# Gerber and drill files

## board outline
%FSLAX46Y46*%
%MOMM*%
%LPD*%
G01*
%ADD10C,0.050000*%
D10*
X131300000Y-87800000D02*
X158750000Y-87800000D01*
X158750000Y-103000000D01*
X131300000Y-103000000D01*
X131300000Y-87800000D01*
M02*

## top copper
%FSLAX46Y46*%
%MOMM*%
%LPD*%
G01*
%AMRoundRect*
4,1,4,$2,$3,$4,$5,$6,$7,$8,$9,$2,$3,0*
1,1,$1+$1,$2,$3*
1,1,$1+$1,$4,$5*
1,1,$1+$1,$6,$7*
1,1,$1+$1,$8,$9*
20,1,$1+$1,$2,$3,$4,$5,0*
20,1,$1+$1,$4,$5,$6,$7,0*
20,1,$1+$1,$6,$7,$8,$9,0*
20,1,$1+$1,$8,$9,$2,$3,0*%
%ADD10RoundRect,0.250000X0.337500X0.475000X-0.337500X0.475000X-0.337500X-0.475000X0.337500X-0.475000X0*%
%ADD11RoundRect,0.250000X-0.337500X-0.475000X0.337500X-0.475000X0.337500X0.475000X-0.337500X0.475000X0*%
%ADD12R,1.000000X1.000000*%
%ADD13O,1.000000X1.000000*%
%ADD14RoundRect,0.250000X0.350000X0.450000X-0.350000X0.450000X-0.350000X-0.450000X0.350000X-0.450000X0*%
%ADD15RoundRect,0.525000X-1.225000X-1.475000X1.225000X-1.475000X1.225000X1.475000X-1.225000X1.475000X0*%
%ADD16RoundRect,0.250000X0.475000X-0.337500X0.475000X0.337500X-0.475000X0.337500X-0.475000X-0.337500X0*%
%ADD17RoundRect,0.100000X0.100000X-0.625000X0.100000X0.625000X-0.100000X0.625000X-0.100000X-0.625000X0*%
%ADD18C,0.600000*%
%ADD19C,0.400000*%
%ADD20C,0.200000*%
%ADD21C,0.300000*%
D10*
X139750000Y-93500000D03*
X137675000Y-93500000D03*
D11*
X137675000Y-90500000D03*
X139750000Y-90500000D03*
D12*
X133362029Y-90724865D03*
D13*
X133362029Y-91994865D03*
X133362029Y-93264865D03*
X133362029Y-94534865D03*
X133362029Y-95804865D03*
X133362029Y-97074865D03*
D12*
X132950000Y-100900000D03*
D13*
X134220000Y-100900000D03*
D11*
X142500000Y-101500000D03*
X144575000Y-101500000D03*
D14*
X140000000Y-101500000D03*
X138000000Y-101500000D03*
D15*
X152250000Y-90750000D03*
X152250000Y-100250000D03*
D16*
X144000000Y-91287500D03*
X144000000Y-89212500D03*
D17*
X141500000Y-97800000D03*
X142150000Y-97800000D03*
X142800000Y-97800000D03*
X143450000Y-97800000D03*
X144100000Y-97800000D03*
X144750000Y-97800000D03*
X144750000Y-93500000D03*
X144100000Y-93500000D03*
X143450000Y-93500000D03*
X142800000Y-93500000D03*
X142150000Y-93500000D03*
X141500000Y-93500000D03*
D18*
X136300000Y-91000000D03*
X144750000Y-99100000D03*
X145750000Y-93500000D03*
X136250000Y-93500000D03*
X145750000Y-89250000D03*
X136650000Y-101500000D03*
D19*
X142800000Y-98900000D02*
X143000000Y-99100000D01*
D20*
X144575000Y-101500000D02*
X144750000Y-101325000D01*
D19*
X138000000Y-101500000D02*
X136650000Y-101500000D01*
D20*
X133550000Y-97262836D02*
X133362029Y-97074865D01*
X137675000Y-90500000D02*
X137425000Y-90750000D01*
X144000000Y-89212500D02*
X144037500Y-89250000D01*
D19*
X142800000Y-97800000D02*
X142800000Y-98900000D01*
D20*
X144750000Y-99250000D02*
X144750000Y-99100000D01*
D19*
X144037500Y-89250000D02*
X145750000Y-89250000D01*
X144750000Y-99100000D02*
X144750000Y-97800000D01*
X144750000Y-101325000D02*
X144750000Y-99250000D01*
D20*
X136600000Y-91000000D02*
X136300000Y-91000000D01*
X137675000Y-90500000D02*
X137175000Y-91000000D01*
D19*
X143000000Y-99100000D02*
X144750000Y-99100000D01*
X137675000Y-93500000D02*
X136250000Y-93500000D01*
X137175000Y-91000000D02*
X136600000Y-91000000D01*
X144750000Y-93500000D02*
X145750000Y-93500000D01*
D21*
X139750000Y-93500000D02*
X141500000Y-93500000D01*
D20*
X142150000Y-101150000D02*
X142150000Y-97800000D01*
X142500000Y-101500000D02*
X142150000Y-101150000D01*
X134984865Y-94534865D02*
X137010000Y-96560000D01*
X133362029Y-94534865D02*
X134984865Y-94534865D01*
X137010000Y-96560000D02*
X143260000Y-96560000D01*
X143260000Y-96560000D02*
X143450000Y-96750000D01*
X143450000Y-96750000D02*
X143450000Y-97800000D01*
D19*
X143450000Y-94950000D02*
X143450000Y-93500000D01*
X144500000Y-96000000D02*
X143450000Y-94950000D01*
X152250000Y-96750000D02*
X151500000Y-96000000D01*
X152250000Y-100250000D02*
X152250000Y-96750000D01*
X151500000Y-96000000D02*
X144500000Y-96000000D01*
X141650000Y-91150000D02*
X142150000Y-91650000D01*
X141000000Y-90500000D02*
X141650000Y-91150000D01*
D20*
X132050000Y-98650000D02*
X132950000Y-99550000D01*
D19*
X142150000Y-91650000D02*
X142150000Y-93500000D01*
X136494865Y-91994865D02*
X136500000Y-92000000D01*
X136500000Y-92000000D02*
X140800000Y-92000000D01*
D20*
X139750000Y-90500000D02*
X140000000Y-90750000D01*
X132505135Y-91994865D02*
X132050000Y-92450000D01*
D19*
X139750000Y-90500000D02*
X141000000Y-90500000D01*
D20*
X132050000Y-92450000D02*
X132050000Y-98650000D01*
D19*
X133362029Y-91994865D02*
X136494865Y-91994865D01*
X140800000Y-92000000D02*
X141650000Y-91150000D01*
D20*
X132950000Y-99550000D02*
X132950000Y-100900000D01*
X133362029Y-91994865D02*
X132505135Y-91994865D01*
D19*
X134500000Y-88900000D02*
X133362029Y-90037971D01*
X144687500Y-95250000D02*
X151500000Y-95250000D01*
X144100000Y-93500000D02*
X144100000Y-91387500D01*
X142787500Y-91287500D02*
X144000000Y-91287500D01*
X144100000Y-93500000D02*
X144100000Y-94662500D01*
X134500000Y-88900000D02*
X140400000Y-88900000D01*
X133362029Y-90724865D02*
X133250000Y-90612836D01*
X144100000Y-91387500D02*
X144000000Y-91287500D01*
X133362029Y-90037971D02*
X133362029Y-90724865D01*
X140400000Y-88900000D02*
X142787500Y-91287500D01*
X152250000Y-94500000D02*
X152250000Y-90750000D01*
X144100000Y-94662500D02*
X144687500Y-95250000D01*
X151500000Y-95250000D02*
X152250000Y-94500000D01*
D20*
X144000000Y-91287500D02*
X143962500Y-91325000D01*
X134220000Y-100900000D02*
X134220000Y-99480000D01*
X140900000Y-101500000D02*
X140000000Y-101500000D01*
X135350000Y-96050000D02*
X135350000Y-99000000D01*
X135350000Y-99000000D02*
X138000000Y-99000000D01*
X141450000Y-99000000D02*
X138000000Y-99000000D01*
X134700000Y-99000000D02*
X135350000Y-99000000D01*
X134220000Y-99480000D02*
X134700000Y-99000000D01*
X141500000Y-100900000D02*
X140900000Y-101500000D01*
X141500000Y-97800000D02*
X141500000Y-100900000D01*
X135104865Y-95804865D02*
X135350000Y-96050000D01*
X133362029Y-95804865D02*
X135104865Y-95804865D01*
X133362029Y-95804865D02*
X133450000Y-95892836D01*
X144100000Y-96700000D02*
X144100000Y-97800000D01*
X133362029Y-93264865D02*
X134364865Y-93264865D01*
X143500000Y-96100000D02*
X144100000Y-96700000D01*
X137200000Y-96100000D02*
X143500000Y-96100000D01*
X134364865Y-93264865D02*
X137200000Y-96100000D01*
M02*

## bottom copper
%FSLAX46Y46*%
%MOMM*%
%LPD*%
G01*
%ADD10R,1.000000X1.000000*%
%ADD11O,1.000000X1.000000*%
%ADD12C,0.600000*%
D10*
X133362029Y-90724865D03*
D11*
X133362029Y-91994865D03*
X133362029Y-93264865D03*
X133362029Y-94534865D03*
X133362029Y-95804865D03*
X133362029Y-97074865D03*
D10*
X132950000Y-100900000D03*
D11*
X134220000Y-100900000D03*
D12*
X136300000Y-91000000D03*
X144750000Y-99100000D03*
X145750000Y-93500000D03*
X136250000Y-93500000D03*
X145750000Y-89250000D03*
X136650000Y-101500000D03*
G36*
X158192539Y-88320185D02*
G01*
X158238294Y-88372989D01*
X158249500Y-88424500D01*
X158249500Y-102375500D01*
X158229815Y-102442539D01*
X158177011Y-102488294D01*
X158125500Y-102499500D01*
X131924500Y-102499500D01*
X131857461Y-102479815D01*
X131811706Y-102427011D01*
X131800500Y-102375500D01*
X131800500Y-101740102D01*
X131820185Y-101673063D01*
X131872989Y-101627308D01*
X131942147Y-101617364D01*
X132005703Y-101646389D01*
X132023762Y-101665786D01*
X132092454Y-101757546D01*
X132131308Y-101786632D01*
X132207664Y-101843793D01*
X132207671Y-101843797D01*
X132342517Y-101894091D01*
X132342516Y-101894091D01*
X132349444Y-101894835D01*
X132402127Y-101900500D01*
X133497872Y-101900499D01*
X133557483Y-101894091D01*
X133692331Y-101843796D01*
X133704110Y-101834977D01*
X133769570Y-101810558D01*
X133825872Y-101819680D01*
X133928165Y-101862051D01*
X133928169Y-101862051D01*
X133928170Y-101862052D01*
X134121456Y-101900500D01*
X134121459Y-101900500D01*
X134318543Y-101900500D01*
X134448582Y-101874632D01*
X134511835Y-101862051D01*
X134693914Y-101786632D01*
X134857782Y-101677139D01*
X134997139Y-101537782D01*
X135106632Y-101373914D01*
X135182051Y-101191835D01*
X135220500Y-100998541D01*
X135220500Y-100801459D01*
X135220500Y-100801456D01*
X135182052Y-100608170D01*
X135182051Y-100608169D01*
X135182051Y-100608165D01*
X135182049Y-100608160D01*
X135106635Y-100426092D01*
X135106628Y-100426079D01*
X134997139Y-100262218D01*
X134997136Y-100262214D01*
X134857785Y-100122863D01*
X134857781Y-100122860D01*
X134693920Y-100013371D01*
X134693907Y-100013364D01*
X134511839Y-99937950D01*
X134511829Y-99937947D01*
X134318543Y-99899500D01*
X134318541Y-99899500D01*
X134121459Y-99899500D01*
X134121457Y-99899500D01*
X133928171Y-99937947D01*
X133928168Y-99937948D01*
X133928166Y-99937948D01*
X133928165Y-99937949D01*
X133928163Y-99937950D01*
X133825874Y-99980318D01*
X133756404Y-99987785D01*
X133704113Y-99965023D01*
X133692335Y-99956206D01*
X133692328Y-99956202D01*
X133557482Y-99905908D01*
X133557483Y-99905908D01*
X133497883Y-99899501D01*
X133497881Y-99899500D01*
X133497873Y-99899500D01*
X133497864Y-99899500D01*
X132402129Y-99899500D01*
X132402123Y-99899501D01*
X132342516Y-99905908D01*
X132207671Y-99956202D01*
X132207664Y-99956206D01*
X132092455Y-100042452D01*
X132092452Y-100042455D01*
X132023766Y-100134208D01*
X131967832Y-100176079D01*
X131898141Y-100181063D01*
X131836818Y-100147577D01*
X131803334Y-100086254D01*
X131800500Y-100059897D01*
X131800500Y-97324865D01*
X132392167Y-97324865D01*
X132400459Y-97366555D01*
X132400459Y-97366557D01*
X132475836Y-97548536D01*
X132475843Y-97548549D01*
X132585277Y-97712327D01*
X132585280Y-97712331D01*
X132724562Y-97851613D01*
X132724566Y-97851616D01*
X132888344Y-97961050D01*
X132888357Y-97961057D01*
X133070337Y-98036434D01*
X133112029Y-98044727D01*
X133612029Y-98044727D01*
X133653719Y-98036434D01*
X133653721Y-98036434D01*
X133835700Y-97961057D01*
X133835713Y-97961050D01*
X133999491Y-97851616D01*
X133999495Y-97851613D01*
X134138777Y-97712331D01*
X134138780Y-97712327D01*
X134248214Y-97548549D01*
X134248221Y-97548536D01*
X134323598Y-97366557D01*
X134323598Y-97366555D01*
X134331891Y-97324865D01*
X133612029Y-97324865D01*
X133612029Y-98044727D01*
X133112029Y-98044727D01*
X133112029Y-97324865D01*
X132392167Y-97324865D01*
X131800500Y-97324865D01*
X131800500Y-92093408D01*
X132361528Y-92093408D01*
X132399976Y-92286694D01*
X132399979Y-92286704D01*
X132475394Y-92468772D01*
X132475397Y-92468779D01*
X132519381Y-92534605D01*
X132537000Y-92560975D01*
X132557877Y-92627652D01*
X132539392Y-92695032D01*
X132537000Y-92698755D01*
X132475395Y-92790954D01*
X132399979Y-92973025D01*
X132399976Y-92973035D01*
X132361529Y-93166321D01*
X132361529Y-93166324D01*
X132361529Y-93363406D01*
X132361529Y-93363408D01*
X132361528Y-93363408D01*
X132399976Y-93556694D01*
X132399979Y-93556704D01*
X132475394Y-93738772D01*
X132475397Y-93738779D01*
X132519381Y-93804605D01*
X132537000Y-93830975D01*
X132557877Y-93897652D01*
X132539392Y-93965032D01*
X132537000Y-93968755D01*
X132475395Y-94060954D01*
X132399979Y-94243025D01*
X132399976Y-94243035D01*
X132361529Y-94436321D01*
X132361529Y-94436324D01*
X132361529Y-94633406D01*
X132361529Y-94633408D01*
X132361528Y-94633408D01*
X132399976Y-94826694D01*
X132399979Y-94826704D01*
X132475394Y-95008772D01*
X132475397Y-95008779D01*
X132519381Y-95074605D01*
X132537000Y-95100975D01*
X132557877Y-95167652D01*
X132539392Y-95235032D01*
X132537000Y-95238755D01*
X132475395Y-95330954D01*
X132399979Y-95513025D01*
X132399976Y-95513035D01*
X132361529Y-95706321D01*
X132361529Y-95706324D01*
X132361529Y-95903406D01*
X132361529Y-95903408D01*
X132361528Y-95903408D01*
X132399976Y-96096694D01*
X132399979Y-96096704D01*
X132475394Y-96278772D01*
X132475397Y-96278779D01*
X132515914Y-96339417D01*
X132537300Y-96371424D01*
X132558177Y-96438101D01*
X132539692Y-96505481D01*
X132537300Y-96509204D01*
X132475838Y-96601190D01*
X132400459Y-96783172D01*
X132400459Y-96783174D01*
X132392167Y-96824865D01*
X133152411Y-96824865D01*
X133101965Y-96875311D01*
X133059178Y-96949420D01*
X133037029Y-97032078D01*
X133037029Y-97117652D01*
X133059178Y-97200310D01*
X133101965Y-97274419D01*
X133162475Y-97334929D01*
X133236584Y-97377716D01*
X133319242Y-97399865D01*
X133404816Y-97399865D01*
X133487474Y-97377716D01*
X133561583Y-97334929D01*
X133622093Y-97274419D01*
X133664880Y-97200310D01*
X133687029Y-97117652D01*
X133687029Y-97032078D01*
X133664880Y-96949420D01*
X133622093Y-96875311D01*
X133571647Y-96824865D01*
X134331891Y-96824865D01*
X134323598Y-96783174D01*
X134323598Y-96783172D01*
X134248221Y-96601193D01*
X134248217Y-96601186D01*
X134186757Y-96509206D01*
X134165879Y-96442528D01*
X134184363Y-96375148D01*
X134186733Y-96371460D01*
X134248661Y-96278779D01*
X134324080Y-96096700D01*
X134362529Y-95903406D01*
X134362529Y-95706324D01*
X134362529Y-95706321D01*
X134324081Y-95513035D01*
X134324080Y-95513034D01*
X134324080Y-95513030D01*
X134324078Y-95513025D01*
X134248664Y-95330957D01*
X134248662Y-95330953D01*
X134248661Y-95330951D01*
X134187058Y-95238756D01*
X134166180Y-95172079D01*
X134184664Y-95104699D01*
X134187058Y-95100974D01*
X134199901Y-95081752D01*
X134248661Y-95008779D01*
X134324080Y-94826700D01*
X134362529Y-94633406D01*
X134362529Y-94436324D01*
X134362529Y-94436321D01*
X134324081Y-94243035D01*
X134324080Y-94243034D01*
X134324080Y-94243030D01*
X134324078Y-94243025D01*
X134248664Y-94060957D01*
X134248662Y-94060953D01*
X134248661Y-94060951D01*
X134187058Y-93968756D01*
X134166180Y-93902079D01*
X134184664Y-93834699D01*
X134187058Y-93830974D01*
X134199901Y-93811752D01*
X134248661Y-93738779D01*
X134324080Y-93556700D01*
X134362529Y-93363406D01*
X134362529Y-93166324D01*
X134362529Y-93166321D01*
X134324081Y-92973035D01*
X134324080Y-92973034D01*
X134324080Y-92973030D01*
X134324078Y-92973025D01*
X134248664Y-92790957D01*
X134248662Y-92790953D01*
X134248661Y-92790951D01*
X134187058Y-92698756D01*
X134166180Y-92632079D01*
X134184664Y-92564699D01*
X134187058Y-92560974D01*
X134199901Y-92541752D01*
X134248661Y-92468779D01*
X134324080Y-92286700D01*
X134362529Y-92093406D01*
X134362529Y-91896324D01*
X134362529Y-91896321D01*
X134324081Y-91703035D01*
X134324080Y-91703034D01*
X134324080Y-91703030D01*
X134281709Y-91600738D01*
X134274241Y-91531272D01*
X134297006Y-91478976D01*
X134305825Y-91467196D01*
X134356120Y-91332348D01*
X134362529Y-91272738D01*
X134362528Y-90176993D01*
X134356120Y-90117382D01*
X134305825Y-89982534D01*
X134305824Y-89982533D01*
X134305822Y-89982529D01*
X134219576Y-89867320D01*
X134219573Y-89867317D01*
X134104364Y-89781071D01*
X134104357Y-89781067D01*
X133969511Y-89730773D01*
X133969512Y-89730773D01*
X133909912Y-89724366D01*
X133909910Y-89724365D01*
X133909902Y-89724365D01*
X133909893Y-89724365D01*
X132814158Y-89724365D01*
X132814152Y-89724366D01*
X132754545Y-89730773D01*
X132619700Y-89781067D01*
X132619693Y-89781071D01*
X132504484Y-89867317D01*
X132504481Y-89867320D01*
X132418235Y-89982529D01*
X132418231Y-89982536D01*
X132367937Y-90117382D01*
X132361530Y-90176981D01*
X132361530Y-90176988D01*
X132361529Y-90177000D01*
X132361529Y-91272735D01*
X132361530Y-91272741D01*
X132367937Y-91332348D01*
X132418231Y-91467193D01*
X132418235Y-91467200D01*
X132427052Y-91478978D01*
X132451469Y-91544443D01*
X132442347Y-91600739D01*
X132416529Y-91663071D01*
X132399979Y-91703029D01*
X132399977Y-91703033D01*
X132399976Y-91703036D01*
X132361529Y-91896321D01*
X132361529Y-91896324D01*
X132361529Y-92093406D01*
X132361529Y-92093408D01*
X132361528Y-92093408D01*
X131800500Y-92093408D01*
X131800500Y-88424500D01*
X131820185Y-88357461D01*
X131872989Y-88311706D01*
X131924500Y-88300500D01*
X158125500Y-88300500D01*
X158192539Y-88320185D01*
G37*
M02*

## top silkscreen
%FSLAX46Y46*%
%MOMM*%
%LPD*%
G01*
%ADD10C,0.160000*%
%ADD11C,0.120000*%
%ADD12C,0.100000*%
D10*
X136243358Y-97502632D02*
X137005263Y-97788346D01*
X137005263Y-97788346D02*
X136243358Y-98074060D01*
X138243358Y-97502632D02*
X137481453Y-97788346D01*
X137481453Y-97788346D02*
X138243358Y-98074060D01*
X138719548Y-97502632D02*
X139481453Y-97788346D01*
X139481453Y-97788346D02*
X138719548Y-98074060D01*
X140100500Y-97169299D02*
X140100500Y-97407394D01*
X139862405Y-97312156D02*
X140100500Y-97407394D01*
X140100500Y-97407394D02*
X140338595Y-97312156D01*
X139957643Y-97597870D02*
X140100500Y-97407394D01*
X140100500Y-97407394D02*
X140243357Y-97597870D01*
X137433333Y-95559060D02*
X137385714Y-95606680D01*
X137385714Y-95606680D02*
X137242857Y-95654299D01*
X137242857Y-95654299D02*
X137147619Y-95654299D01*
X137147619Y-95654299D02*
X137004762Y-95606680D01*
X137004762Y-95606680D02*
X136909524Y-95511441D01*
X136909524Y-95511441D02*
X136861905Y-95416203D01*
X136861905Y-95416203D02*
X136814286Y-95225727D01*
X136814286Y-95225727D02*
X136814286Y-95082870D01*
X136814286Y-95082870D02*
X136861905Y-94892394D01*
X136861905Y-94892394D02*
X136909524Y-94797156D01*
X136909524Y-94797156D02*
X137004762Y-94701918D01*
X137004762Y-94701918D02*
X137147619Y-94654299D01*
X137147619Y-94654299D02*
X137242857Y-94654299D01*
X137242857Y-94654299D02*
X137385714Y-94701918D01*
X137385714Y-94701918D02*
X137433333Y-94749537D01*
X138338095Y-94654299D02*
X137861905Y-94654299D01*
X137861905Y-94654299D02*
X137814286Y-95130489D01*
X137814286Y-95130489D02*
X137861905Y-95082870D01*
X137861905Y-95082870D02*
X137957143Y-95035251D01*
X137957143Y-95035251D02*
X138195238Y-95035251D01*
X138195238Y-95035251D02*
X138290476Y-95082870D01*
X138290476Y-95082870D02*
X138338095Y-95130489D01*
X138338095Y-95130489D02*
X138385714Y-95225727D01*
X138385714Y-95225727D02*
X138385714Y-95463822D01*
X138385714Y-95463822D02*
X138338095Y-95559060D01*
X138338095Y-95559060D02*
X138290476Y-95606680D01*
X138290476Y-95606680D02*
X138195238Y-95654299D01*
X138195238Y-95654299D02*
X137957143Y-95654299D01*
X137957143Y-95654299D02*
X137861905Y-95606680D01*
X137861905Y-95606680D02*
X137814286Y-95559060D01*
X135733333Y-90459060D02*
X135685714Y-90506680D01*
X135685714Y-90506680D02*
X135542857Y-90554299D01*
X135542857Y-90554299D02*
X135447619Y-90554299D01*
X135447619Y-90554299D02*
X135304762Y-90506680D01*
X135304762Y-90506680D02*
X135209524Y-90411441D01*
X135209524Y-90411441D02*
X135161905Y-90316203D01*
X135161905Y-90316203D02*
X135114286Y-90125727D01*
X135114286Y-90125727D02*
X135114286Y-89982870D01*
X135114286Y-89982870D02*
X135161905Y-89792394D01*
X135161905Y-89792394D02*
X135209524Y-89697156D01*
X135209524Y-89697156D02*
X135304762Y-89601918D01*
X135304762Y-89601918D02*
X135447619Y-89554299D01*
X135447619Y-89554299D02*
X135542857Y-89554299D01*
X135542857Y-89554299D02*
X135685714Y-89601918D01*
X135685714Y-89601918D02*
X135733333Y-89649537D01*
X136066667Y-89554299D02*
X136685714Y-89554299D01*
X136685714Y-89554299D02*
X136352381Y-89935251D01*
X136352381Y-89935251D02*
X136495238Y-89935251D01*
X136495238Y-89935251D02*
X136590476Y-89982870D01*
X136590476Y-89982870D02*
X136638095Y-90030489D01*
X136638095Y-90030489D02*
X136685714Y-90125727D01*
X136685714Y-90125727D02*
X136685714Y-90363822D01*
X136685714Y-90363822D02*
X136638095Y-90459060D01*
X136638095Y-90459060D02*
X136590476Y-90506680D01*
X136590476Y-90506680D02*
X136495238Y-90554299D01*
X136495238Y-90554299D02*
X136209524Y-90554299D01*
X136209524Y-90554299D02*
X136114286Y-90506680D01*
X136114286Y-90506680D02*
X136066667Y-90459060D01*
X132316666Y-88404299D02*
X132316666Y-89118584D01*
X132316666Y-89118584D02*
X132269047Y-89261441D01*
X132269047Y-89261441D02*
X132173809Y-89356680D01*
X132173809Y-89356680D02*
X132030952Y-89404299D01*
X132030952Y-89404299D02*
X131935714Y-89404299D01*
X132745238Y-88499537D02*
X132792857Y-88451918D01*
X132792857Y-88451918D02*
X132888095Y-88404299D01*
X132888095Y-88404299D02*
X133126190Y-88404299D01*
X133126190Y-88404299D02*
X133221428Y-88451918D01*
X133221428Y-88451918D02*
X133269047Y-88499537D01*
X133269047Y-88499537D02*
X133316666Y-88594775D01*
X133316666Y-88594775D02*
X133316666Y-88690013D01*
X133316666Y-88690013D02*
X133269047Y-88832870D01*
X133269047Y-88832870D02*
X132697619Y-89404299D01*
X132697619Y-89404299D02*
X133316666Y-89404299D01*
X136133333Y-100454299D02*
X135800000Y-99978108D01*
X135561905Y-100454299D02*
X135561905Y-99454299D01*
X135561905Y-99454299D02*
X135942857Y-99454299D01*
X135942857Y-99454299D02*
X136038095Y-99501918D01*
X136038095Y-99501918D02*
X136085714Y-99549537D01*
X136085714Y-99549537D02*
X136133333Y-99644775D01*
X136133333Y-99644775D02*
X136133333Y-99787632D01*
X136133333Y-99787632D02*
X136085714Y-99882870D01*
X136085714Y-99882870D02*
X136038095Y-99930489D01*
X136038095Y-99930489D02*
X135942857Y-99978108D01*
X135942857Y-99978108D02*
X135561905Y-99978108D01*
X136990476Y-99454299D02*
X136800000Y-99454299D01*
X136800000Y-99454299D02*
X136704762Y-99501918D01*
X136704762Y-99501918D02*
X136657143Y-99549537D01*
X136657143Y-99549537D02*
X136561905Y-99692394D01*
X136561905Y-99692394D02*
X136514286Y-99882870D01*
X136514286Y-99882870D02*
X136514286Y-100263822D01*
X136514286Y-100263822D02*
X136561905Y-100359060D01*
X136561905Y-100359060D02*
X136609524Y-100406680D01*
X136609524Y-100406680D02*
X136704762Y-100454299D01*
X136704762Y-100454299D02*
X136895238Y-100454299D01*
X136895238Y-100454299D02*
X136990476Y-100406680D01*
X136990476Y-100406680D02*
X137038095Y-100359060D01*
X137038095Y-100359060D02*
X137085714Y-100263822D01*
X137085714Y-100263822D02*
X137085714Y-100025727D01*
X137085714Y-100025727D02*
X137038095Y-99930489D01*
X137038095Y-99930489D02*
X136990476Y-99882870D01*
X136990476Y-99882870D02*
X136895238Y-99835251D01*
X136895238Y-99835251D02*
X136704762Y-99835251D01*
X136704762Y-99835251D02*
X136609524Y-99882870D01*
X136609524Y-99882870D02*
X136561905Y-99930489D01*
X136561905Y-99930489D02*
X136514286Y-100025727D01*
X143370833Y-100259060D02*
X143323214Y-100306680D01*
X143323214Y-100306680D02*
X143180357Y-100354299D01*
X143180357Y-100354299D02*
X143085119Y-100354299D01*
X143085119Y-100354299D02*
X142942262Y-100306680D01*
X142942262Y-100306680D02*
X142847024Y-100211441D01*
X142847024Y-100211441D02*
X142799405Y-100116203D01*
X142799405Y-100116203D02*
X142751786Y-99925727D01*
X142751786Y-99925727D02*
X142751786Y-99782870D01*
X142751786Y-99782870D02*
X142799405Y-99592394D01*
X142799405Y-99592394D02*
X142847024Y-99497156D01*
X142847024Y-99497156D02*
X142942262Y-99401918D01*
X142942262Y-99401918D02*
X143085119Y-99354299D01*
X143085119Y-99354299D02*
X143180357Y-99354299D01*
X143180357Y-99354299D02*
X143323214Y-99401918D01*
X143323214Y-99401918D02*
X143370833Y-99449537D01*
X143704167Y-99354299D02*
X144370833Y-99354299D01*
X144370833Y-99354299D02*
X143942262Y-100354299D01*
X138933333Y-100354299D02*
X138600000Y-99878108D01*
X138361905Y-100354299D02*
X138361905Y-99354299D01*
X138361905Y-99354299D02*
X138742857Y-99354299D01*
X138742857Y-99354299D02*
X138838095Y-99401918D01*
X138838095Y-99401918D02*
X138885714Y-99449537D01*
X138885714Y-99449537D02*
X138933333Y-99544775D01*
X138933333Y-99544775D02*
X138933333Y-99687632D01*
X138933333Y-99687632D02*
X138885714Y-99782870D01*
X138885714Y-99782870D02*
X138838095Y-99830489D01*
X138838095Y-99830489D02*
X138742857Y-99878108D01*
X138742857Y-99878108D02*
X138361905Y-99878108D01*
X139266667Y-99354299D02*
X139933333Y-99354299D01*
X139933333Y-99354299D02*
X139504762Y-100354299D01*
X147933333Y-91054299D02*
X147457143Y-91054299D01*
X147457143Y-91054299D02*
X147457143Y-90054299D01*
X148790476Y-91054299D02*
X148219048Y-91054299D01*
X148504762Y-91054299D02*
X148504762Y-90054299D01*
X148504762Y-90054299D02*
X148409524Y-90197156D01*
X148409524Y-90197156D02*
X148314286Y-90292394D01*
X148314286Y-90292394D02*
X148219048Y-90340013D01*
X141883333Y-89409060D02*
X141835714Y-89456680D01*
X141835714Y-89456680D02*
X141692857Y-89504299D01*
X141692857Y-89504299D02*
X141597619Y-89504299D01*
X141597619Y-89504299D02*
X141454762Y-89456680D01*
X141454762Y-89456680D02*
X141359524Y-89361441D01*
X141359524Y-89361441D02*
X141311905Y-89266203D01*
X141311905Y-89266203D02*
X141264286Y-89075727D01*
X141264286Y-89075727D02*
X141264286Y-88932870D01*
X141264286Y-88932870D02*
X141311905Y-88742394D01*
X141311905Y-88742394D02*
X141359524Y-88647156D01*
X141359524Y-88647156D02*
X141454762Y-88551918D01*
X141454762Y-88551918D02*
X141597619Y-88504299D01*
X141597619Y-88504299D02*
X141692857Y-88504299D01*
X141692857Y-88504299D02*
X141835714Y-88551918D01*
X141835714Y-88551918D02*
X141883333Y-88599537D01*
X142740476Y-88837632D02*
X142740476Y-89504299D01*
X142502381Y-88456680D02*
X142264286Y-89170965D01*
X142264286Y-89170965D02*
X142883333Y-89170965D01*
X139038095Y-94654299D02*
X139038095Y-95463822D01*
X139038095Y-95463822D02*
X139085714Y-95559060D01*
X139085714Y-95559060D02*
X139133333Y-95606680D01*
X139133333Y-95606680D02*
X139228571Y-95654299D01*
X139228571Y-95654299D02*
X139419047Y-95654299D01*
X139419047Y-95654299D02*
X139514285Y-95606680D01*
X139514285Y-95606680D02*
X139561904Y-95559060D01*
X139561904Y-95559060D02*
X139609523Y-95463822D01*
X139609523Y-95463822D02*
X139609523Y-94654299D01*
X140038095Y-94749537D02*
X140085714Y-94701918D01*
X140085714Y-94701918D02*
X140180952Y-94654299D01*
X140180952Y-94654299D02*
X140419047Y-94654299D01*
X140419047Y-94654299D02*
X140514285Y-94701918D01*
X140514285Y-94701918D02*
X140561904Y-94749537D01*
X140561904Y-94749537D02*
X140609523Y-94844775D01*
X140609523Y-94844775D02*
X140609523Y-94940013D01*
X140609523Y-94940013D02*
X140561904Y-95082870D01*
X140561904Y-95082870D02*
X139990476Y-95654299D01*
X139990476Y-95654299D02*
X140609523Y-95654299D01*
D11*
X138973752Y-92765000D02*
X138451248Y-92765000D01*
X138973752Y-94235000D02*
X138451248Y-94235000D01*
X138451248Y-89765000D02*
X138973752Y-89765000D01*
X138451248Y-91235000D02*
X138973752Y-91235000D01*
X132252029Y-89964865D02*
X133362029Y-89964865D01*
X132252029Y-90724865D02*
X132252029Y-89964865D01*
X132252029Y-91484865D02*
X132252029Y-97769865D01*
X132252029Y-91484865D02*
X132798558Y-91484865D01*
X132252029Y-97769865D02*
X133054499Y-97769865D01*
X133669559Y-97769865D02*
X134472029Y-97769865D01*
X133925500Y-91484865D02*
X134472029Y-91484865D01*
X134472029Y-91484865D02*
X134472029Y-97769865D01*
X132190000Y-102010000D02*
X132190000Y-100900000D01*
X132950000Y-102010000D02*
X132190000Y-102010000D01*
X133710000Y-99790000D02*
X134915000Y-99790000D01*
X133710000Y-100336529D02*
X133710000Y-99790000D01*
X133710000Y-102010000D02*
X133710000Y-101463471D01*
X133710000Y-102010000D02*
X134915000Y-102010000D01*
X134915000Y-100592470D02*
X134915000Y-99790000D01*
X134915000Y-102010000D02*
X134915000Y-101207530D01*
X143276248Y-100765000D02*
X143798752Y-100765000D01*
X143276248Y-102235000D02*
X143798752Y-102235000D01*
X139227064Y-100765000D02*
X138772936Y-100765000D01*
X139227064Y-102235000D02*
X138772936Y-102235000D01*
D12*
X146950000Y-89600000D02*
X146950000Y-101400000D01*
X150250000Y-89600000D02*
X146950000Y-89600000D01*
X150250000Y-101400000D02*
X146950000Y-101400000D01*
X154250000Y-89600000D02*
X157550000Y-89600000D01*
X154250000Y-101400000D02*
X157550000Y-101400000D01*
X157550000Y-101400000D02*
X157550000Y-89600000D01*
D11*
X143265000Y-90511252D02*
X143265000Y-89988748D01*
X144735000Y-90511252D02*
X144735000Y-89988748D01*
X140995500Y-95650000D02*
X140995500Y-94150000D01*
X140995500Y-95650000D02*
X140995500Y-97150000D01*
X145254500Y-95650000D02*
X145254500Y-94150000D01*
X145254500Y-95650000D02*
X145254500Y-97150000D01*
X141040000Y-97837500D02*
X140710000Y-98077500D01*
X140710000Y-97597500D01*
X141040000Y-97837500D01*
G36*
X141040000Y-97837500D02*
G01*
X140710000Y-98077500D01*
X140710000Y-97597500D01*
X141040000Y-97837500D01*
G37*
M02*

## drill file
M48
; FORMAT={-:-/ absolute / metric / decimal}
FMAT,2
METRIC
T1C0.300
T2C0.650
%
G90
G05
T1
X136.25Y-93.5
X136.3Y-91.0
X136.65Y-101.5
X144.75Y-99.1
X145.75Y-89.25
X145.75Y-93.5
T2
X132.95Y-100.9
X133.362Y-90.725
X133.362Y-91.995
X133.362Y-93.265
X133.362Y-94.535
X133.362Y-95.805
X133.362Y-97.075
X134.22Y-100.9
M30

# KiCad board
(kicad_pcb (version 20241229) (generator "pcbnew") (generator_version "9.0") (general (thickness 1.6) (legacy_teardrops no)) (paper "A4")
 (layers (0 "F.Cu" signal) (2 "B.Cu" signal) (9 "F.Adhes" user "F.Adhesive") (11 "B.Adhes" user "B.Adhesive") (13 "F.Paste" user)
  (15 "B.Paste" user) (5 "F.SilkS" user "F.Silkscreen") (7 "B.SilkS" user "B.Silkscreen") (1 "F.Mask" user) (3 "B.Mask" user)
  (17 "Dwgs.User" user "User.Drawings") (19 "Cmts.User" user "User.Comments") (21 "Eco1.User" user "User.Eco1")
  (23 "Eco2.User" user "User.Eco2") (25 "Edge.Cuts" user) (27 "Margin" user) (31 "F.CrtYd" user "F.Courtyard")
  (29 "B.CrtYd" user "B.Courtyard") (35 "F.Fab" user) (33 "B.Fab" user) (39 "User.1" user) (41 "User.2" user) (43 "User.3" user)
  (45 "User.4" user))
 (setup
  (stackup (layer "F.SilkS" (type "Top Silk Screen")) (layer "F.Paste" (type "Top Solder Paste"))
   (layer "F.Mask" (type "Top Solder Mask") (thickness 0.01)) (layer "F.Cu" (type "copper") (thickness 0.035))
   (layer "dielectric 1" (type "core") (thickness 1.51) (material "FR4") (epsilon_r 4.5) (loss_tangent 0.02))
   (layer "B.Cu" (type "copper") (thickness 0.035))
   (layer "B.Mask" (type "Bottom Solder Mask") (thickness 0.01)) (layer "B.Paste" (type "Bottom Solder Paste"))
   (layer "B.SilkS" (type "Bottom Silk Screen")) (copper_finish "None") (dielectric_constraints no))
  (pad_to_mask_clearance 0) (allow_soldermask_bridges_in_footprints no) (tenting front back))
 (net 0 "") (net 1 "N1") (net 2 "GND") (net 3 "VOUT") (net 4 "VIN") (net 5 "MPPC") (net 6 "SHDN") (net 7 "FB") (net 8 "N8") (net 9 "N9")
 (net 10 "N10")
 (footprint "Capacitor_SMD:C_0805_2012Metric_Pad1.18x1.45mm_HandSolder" (layer "F.Cu") (at 138.7125 93.5 180)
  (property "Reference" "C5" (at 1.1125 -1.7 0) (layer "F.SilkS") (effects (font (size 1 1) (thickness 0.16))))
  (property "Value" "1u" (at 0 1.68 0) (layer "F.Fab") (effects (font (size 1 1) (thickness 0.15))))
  (fp_line (start -0.261252 0.735) (end 0.261252 0.735) (stroke (width 0.12) (type solid)) (layer "F.SilkS"))
  (fp_line (start -0.261252 -0.735) (end 0.261252 -0.735) (stroke (width 0.12) (type solid)) (layer "F.SilkS"))
  (pad "1" smd roundrect (at -1.0375 0 180) (size 1.175 1.45) (layers "F.Cu" "F.Mask" "F.Paste") (roundrect_rratio 0.212766) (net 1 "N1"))
  (pad "2" smd roundrect (at 1.0375 0 180) (size 1.175 1.45) (layers "F.Cu" "F.Mask" "F.Paste") (roundrect_rratio 0.212766) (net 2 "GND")))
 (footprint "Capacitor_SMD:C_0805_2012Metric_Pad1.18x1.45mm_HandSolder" (layer "F.Cu") (at 138.7125 90.5)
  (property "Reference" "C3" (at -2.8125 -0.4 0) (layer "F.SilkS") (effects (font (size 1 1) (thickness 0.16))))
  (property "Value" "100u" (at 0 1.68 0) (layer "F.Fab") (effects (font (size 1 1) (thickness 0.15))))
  (fp_line (start -0.261252 -0.735) (end 0.261252 -0.735) (stroke (width 0.12) (type solid)) (layer "F.SilkS"))
  (fp_line (start -0.261252 0.735) (end 0.261252 0.735) (stroke (width 0.12) (type solid)) (layer "F.SilkS"))
  (pad "1" smd roundrect (at -1.0375 0) (size 1.175 1.45) (layers "F.Cu" "F.Mask" "F.Paste") (roundrect_rratio 0.212766) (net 2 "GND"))
  (pad "2" smd roundrect (at 1.0375 0) (size 1.175 1.45) (layers "F.Cu" "F.Mask" "F.Paste") (roundrect_rratio 0.212766) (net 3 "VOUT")))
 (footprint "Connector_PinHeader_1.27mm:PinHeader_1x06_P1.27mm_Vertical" (layer "F.Cu") (at 133.362029 90.724865)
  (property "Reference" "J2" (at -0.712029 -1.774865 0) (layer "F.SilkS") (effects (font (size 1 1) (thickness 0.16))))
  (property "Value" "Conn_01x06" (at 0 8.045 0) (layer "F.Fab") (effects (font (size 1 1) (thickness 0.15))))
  (fp_line (start -1.11 -0.76) (end 0 -0.76) (stroke (width 0.12) (type solid)) (layer "F.SilkS"))
  (fp_line (start -1.11 0) (end -1.11 -0.76) (stroke (width 0.12) (type solid)) (layer "F.SilkS"))
  (fp_line (start -1.11 0.76) (end -1.11 7.045) (stroke (width 0.12) (type solid)) (layer "F.SilkS"))
  (fp_line (start -1.11 0.76) (end -0.563471 0.76) (stroke (width 0.12) (type solid)) (layer "F.SilkS"))
  (fp_line (start -1.11 7.045) (end -0.30753 7.045) (stroke (width 0.12) (type solid)) (layer "F.SilkS"))
  (fp_line (start 0.30753 7.045) (end 1.11 7.045) (stroke (width 0.12) (type solid)) (layer "F.SilkS"))
  (fp_line (start 0.563471 0.76) (end 1.11 0.76) (stroke (width 0.12) (type solid)) (layer "F.SilkS"))
  (fp_line (start 1.11 0.76) (end 1.11 7.045) (stroke (width 0.12) (type solid)) (layer "F.SilkS"))
  (pad "1" thru_hole rect (at 0 0) (size 1 1) (drill 0.65) (layers "*.Cu" "*.Mask") (remove_unused_layers no) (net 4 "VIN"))
  (pad "2" thru_hole oval (at 0 1.27) (size 1 1) (drill 0.65) (layers "*.Cu" "*.Mask") (remove_unused_layers no) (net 3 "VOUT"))
  (pad "3" thru_hole oval (at 0 2.54) (size 1 1) (drill 0.65) (layers "*.Cu" "*.Mask") (remove_unused_layers no) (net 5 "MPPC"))
  (pad "4" thru_hole oval (at 0 3.81) (size 1 1) (drill 0.65) (layers "*.Cu" "*.Mask") (remove_unused_layers no) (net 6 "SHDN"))
  (pad "5" thru_hole oval (at 0 5.08) (size 1 1) (drill 0.65) (layers "*.Cu" "*.Mask") (remove_unused_layers no) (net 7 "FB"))
  (pad "6" thru_hole oval (at 0 6.35) (size 1 1) (drill 0.65) (layers "*.Cu" "*.Mask") (remove_unused_layers no) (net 2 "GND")))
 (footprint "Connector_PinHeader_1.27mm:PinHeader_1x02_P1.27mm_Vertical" (layer "F.Cu") (at 132.95 100.9 90)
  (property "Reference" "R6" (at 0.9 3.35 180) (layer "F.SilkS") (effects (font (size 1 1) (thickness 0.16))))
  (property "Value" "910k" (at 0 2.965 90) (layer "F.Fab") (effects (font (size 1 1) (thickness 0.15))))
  (fp_line (start -1.11 -0.76) (end 0 -0.76) (stroke (width 0.12) (type solid)) (layer "F.SilkS"))
  (fp_line (start -1.11 0) (end -1.11 -0.76) (stroke (width 0.12) (type solid)) (layer "F.SilkS"))
  (fp_line (start 1.11 0.76) (end 1.11 1.965) (stroke (width 0.12) (type solid)) (layer "F.SilkS"))
  (fp_line (start 0.563471 0.76) (end 1.11 0.76) (stroke (width 0.12) (type solid)) (layer "F.SilkS"))
  (fp_line (start -1.11 0.76) (end -0.563471 0.76) (stroke (width 0.12) (type solid)) (layer "F.SilkS"))
  (fp_line (start -1.11 0.76) (end -1.11 1.965) (stroke (width 0.12) (type solid)) (layer "F.SilkS"))
  (fp_line (start 0.30753 1.965) (end 1.11 1.965) (stroke (width 0.12) (type solid)) (layer "F.SilkS"))
  (fp_line (start -1.11 1.965) (end -0.30753 1.965) (stroke (width 0.12) (type solid)) (layer "F.SilkS"))
  (pad "1" thru_hole rect (at 0 0 90) (size 1 1) (drill 0.65) (layers "*.Cu" "*.Mask") (remove_unused_layers no) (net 3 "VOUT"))
  (pad "2" thru_hole oval (at 0 1.27 90) (size 1 1) (drill 0.65) (layers "*.Cu" "*.Mask") (remove_unused_layers no) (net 7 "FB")))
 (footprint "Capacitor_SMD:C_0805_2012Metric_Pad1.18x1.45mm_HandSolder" (layer "F.Cu") (at 143.5375 101.5)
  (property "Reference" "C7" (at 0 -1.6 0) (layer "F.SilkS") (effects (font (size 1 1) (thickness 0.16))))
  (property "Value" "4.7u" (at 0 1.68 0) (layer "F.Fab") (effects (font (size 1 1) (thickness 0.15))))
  (fp_line (start -0.261252 -0.735) (end 0.261252 -0.735) (stroke (width 0.12) (type solid)) (layer "F.SilkS"))
  (fp_line (start -0.261252 0.735) (end 0.261252 0.735) (stroke (width 0.12) (type solid)) (layer "F.SilkS"))
  (pad "1" smd roundrect (at -1.0375 0) (size 1.175 1.45) (layers "F.Cu" "F.Mask" "F.Paste") (roundrect_rratio 0.212766) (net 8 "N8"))
  (pad "2" smd roundrect (at 1.0375 0) (size 1.175 1.45) (layers "F.Cu" "F.Mask" "F.Paste") (roundrect_rratio 0.212766) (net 2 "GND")))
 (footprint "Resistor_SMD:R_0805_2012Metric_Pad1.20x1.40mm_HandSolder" (layer "F.Cu") (at 139 101.5 180)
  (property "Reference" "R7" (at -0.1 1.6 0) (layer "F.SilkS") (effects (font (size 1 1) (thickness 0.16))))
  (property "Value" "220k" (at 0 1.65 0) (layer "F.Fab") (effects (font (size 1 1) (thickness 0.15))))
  (fp_line (start -0.227064 0.735) (end 0.227064 0.735) (stroke (width 0.12) (type solid)) (layer "F.SilkS"))
  (fp_line (start -0.227064 -0.735) (end 0.227064 -0.735) (stroke (width 0.12) (type solid)) (layer "F.SilkS"))
  (pad "1" smd roundrect (at -1 0 180) (size 1.2 1.4) (layers "F.Cu" "F.Mask" "F.Paste") (roundrect_rratio 0.208333) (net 7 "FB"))
  (pad "2" smd roundrect (at 1 0 180) (size 1.2 1.4) (layers "F.Cu" "F.Mask" "F.Paste") (roundrect_rratio 0.208333) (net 2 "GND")))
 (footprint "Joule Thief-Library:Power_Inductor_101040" (layer "F.Cu") (at 152.25 95.5 -90)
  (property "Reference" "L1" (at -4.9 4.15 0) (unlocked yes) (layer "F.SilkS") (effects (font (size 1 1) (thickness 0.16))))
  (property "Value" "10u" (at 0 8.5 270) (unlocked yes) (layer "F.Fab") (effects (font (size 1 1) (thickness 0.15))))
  (fp_line (start -5.9 5.3) (end 5.9 5.3) (stroke (width 0.1) (type default)) (layer "F.SilkS"))
  (fp_line (start -5.9 2) (end -5.9 5.3) (stroke (width 0.1) (type default)) (layer "F.SilkS"))
  (fp_line (start 5.9 2) (end 5.9 5.3) (stroke (width 0.1) (type default)) (layer "F.SilkS"))
  (fp_line (start -5.9 -2) (end -5.9 -5.3) (stroke (width 0.1) (type default)) (layer "F.SilkS"))
  (fp_line (start 5.9 -2) (end 5.9 -5.3) (stroke (width 0.1) (type default)) (layer "F.SilkS"))
  (fp_line (start 5.9 -5.3) (end -5.9 -5.3) (stroke (width 0.1) (type default)) (layer "F.SilkS"))
  (pad "1" smd roundrect (at -4.75 0) (size 3.5 4) (layers "F.Cu" "F.Mask" "F.Paste") (roundrect_rratio 0.15) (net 4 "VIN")
   (thermal_bridge_angle 45))
  (pad "2" smd roundrect (at 4.75 0) (size 3.5 4) (layers "F.Cu" "F.Mask" "F.Paste") (roundrect_rratio 0.15) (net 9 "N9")
   (thermal_bridge_angle 45)))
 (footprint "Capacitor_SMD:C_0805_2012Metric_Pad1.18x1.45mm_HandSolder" (layer "F.Cu") (at 144 90.25 90)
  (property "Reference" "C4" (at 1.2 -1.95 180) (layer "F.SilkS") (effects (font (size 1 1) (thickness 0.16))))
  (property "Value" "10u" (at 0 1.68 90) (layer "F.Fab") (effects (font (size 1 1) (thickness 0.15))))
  (fp_line (start -0.261252 -0.735) (end 0.261252 -0.735) (stroke (width 0.12) (type solid)) (layer "F.SilkS"))
  (fp_line (start -0.261252 0.735) (end 0.261252 0.735) (stroke (width 0.12) (type solid)) (layer "F.SilkS"))
  (pad "1" smd roundrect (at -1.0375 0 90) (size 1.175 1.45) (layers "F.Cu" "F.Mask" "F.Paste") (roundrect_rratio 0.212766) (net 4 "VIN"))
  (pad "2" smd roundrect (at 1.0375 0 90) (size 1.175 1.45) (layers "F.Cu" "F.Mask" "F.Paste") (roundrect_rratio 0.212766) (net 2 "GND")))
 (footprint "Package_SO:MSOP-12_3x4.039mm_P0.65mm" (layer "F.Cu") (at 143.125 95.65 90)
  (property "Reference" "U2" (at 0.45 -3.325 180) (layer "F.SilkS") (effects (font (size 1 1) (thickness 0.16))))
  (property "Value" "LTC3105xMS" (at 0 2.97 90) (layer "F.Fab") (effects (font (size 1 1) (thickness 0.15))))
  (fp_line (start 0 -2.1295) (end 1.5 -2.1295) (stroke (width 0.12) (type solid)) (layer "F.SilkS"))
  (fp_line (start 0 -2.1295) (end -1.5 -2.1295) (stroke (width 0.12) (type solid)) (layer "F.SilkS"))
  (fp_line (start 0 2.1295) (end 1.5 2.1295) (stroke (width 0.12) (type solid)) (layer "F.SilkS"))
  (fp_line (start 0 2.1295) (end -1.5 2.1295) (stroke (width 0.12) (type solid)) (layer "F.SilkS"))
  (fp_poly
   (pts (xy -2.1875 -2.085) (xy -2.4275 -2.415) (xy -1.9475 -2.415) (xy -2.1875 -2.085)) (stroke (width 0.12) (type solid)) (fill yes)
   (layer "F.SilkS"))
  (pad "1" smd roundrect (at -2.15 -1.625 90) (size 1.45 0.4) (layers "F.Cu" "F.Mask" "F.Paste") (roundrect_rratio 0.25) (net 7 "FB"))
  (pad "2" smd roundrect (at -2.15 -0.975 90) (size 1.45 0.4) (layers "F.Cu" "F.Mask" "F.Paste") (roundrect_rratio 0.25) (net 8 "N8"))
  (pad "3" smd roundrect (at -2.15 -0.325 90) (size 1.45 0.4) (layers "F.Cu" "F.Mask" "F.Paste") (roundrect_rratio 0.25) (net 2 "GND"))
  (pad "4" smd roundrect (at -2.15 0.325 90) (size 1.45 0.4) (layers "F.Cu" "F.Mask" "F.Paste") (roundrect_rratio 0.25) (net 6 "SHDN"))
  (pad "5" smd roundrect (at -2.15 0.975 90) (size 1.45 0.4) (layers "F.Cu" "F.Mask" "F.Paste") (roundrect_rratio 0.25) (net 5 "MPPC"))
  (pad "6" smd roundrect (at -2.15 1.625 90) (size 1.45 0.4) (layers "F.Cu" "F.Mask" "F.Paste") (roundrect_rratio 0.25) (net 2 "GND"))
  (pad "7" smd roundrect (at 2.15 1.625 90) (size 1.45 0.4) (layers "F.Cu" "F.Mask" "F.Paste") (roundrect_rratio 0.25) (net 2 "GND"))
  (pad "8" smd roundrect (at 2.15 0.975 90) (size 1.45 0.4) (layers "F.Cu" "F.Mask" "F.Paste") (roundrect_rratio 0.25) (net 4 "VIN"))
  (pad "9" smd roundrect (at 2.15 0.325 90) (size 1.45 0.4) (layers "F.Cu" "F.Mask" "F.Paste") (roundrect_rratio 0.25) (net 9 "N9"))
  (pad "10" smd roundrect (at 2.15 -0.325 90) (size 1.45 0.4) (layers "F.Cu" "F.Mask" "F.Paste") (roundrect_rratio 0.25) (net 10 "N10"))
  (pad "11" smd roundrect (at 2.15 -0.975 90) (size 1.45 0.4) (layers "F.Cu" "F.Mask" "F.Paste") (roundrect_rratio 0.25) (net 3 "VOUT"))
  (pad "12" smd roundrect (at 2.15 -1.625 90) (size 1.45 0.4) (layers "F.Cu" "F.Mask" "F.Paste") (roundrect_rratio 0.25) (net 1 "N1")))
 (gr_rect (start 131.3 87.8) (end 158.75 103) (stroke (width 0.05) (type default)) (fill no) (layer "Edge.Cuts"))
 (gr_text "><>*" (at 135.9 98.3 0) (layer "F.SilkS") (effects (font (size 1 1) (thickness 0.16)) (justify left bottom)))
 (segment (start 142.8 98.9) (end 143 99.1) (width 0.4) (layer "F.Cu") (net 2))
 (segment (start 144.575 101.5) (end 144.75 101.325) (width 0.2) (layer "F.Cu") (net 2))
 (segment (start 138 101.5) (end 136.65 101.5) (width 0.4) (layer "F.Cu") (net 2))
 (segment (start 133.55 97.262836) (end 133.362029 97.074865) (width 0.2) (layer "F.Cu") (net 2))
 (segment (start 137.675 90.5) (end 137.425 90.75) (width 0.2) (layer "F.Cu") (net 2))
 (segment (start 144 89.2125) (end 144.0375 89.25) (width 0.2) (layer "F.Cu") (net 2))
 (segment (start 142.8 97.8) (end 142.8 98.9) (width 0.4) (layer "F.Cu") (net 2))
 (segment (start 144.75 99.25) (end 144.75 99.1) (width 0.2) (layer "F.Cu") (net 2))
 (segment (start 144.0375 89.25) (end 145.75 89.25) (width 0.4) (layer "F.Cu") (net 2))
 (segment (start 144.75 99.1) (end 144.75 97.8) (width 0.4) (layer "F.Cu") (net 2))
 (segment (start 144.75 101.325) (end 144.75 99.25) (width 0.4) (layer "F.Cu") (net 2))
 (segment (start 136.6 91) (end 136.3 91) (width 0.2) (layer "F.Cu") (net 2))
 (segment (start 137.675 90.5) (end 137.175 91) (width 0.2) (layer "F.Cu") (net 2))
 (segment (start 143 99.1) (end 144.75 99.1) (width 0.4) (layer "F.Cu") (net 2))
 (segment (start 137.675 93.5) (end 136.25 93.5) (width 0.4) (layer "F.Cu") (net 2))
 (segment (start 137.175 91) (end 136.6 91) (width 0.4) (layer "F.Cu") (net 2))
 (segment (start 144.75 93.5) (end 145.75 93.5) (width 0.4) (layer "F.Cu") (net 2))
 (via (at 136.3 91) (size 0.6) (drill 0.3) (layers "F.Cu" "B.Cu") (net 2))
 (via (at 144.75 99.1) (size 0.6) (drill 0.3) (layers "F.Cu" "B.Cu") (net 2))
 (via (at 145.75 93.5) (size 0.6) (drill 0.3) (layers "F.Cu" "B.Cu") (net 2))
 (via (at 136.25 93.5) (size 0.6) (drill 0.3) (layers "F.Cu" "B.Cu") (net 2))
 (via (at 145.75 89.25) (size 0.6) (drill 0.3) (layers "F.Cu" "B.Cu") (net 2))
 (via (at 136.65 101.5) (size 0.6) (drill 0.3) (layers "F.Cu" "B.Cu") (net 2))
 (segment (start 139.75 93.5) (end 141.5 93.5) (width 0.3) (layer "F.Cu") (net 1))
 (segment (start 142.15 101.15) (end 142.15 97.8) (width 0.2) (layer "F.Cu") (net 8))
 (segment (start 142.5 101.5) (end 142.15 101.15) (width 0.2) (layer "F.Cu") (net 8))
 (segment (start 134.984865 94.534865) (end 137.01 96.56) (width 0.2) (layer "F.Cu") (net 6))
 (segment (start 133.362029 94.534865) (end 134.984865 94.534865) (width 0.2) (layer "F.Cu") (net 6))
 (segment (start 137.01 96.56) (end 143.26 96.56) (width 0.2) (layer "F.Cu") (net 6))
 (segment (start 143.26 96.56) (end 143.45 96.75) (width 0.2) (layer "F.Cu") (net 6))
 (segment (start 143.45 96.75) (end 143.45 97.8) (width 0.2) (layer "F.Cu") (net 6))
 (segment (start 143.45 94.95) (end 143.45 93.5) (width 0.4) (layer "F.Cu") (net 9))
 (segment (start 144.5 96) (end 143.45 94.95) (width 0.4) (layer "F.Cu") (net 9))
 (segment (start 152.25 96.75) (end 151.5 96) (width 0.4) (layer "F.Cu") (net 9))
 (segment (start 152.25 100.25) (end 152.25 96.75) (width 0.4) (layer "F.Cu") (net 9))
 (segment (start 151.5 96) (end 144.5 96) (width 0.4) (layer "F.Cu") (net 9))
 (segment (start 141.65 91.15) (end 142.15 91.65) (width 0.4) (layer "F.Cu") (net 3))
 (segment (start 141 90.5) (end 141.65 91.15) (width 0.4) (layer "F.Cu") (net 3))
 (segment (start 132.05 98.65) (end 132.95 99.55) (width 0.2) (layer "F.Cu") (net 3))
 (segment (start 142.15 91.65) (end 142.15 93.5) (width 0.4) (layer "F.Cu") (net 3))
 (segment (start 136.494865 91.994865) (end 136.5 92) (width 0.4) (layer "F.Cu") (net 3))
 (segment (start 136.5 92) (end 140.8 92) (width 0.4) (layer "F.Cu") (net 3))
 (segment (start 139.75 90.5) (end 140 90.75) (width 0.2) (layer "F.Cu") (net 3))
 (segment (start 132.505135 91.994865) (end 132.05 92.45) (width 0.2) (layer "F.Cu") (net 3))
 (segment (start 139.75 90.5) (end 141 90.5) (width 0.4) (layer "F.Cu") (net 3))
 (segment (start 132.05 92.45) (end 132.05 98.65) (width 0.2) (layer "F.Cu") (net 3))
 (segment (start 133.362029 91.994865) (end 136.494865 91.994865) (width 0.4) (layer "F.Cu") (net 3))
 (segment (start 140.8 92) (end 141.65 91.15) (width 0.4) (layer "F.Cu") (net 3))
 (segment (start 132.95 99.55) (end 132.95 100.9) (width 0.2) (layer "F.Cu") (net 3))
 (segment (start 133.362029 91.994865) (end 132.505135 91.994865) (width 0.2) (layer "F.Cu") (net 3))
 (segment (start 134.5 88.9) (end 133.362029 90.037971) (width 0.4) (layer "F.Cu") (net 4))
 (segment (start 144.6875 95.25) (end 151.5 95.25) (width 0.4) (layer "F.Cu") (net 4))
 (segment (start 144.1 93.5) (end 144.1 91.3875) (width 0.4) (layer "F.Cu") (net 4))
 (segment (start 142.7875 91.2875) (end 144 91.2875) (width 0.4) (layer "F.Cu") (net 4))
 (segment (start 144.1 93.5) (end 144.1 94.6625) (width 0.4) (layer "F.Cu") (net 4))
 (segment (start 134.5 88.9) (end 140.4 88.9) (width 0.4) (layer "F.Cu") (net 4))
 (segment (start 133.362029 90.724865) (end 133.25 90.612836) (width 0.4) (layer "F.Cu") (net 4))
 (segment (start 144.1 91.3875) (end 144 91.2875) (width 0.4) (layer "F.Cu") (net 4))
 (segment (start 133.362029 90.037971) (end 133.362029 90.724865) (width 0.4) (layer "F.Cu") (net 4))
 (segment (start 140.4 88.9) (end 142.7875 91.2875) (width 0.4) (layer "F.Cu") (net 4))
 (segment (start 152.25 94.5) (end 152.25 90.75) (width 0.4) (layer "F.Cu") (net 4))
 (segment (start 144.1 94.6625) (end 144.6875 95.25) (width 0.4) (layer "F.Cu") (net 4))
 (segment (start 151.5 95.25) (end 152.25 94.5) (width 0.4) (layer "F.Cu") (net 4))
 (segment (start 144 91.2875) (end 143.9625 91.325) (width 0.2) (layer "F.Cu") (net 4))
 (segment (start 134.22 100.9) (end 134.22 99.48) (width 0.2) (layer "F.Cu") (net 7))
 (segment (start 140.9 101.5) (end 140 101.5) (width 0.2) (layer "F.Cu") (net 7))
 (segment (start 135.35 96.05) (end 135.35 99) (width 0.2) (layer "F.Cu") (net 7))
 (segment (start 135.35 99) (end 138 99) (width 0.2) (layer "F.Cu") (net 7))
 (segment (start 141.45 99) (end 138 99) (width 0.2) (layer "F.Cu") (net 7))
 (segment (start 134.7 99) (end 135.35 99) (width 0.2) (layer "F.Cu") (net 7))
 (segment (start 134.22 99.48) (end 134.7 99) (width 0.2) (layer "F.Cu") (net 7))
 (segment (start 141.5 100.9) (end 140.9 101.5) (width 0.2) (layer "F.Cu") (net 7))
 (segment (start 141.5 97.8) (end 141.5 100.9) (width 0.2) (layer "F.Cu") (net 7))
 (segment (start 135.104865 95.804865) (end 135.35 96.05) (width 0.2) (layer "F.Cu") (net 7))
 (segment (start 133.362029 95.804865) (end 135.104865 95.804865) (width 0.2) (layer "F.Cu") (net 7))
 (segment (start 133.362029 95.804865) (end 133.45 95.892836) (width 0.2) (layer "F.Cu") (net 7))
 (segment (start 144.1 96.7) (end 144.1 97.8) (width 0.2) (layer "F.Cu") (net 5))
 (segment (start 133.362029 93.264865) (end 134.364865 93.264865) (width 0.2) (layer "F.Cu") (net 5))
 (segment (start 143.5 96.1) (end 144.1 96.7) (width 0.2) (layer "F.Cu") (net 5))
 (segment (start 137.2 96.1) (end 143.5 96.1) (width 0.2) (layer "F.Cu") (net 5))
 (segment (start 134.364865 93.264865) (end 137.2 96.1) (width 0.2) (layer "F.Cu") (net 5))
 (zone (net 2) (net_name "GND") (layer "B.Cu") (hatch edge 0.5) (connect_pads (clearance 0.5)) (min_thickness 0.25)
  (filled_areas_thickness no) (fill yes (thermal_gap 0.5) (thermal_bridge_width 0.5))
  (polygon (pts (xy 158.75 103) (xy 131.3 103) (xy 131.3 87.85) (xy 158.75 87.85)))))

